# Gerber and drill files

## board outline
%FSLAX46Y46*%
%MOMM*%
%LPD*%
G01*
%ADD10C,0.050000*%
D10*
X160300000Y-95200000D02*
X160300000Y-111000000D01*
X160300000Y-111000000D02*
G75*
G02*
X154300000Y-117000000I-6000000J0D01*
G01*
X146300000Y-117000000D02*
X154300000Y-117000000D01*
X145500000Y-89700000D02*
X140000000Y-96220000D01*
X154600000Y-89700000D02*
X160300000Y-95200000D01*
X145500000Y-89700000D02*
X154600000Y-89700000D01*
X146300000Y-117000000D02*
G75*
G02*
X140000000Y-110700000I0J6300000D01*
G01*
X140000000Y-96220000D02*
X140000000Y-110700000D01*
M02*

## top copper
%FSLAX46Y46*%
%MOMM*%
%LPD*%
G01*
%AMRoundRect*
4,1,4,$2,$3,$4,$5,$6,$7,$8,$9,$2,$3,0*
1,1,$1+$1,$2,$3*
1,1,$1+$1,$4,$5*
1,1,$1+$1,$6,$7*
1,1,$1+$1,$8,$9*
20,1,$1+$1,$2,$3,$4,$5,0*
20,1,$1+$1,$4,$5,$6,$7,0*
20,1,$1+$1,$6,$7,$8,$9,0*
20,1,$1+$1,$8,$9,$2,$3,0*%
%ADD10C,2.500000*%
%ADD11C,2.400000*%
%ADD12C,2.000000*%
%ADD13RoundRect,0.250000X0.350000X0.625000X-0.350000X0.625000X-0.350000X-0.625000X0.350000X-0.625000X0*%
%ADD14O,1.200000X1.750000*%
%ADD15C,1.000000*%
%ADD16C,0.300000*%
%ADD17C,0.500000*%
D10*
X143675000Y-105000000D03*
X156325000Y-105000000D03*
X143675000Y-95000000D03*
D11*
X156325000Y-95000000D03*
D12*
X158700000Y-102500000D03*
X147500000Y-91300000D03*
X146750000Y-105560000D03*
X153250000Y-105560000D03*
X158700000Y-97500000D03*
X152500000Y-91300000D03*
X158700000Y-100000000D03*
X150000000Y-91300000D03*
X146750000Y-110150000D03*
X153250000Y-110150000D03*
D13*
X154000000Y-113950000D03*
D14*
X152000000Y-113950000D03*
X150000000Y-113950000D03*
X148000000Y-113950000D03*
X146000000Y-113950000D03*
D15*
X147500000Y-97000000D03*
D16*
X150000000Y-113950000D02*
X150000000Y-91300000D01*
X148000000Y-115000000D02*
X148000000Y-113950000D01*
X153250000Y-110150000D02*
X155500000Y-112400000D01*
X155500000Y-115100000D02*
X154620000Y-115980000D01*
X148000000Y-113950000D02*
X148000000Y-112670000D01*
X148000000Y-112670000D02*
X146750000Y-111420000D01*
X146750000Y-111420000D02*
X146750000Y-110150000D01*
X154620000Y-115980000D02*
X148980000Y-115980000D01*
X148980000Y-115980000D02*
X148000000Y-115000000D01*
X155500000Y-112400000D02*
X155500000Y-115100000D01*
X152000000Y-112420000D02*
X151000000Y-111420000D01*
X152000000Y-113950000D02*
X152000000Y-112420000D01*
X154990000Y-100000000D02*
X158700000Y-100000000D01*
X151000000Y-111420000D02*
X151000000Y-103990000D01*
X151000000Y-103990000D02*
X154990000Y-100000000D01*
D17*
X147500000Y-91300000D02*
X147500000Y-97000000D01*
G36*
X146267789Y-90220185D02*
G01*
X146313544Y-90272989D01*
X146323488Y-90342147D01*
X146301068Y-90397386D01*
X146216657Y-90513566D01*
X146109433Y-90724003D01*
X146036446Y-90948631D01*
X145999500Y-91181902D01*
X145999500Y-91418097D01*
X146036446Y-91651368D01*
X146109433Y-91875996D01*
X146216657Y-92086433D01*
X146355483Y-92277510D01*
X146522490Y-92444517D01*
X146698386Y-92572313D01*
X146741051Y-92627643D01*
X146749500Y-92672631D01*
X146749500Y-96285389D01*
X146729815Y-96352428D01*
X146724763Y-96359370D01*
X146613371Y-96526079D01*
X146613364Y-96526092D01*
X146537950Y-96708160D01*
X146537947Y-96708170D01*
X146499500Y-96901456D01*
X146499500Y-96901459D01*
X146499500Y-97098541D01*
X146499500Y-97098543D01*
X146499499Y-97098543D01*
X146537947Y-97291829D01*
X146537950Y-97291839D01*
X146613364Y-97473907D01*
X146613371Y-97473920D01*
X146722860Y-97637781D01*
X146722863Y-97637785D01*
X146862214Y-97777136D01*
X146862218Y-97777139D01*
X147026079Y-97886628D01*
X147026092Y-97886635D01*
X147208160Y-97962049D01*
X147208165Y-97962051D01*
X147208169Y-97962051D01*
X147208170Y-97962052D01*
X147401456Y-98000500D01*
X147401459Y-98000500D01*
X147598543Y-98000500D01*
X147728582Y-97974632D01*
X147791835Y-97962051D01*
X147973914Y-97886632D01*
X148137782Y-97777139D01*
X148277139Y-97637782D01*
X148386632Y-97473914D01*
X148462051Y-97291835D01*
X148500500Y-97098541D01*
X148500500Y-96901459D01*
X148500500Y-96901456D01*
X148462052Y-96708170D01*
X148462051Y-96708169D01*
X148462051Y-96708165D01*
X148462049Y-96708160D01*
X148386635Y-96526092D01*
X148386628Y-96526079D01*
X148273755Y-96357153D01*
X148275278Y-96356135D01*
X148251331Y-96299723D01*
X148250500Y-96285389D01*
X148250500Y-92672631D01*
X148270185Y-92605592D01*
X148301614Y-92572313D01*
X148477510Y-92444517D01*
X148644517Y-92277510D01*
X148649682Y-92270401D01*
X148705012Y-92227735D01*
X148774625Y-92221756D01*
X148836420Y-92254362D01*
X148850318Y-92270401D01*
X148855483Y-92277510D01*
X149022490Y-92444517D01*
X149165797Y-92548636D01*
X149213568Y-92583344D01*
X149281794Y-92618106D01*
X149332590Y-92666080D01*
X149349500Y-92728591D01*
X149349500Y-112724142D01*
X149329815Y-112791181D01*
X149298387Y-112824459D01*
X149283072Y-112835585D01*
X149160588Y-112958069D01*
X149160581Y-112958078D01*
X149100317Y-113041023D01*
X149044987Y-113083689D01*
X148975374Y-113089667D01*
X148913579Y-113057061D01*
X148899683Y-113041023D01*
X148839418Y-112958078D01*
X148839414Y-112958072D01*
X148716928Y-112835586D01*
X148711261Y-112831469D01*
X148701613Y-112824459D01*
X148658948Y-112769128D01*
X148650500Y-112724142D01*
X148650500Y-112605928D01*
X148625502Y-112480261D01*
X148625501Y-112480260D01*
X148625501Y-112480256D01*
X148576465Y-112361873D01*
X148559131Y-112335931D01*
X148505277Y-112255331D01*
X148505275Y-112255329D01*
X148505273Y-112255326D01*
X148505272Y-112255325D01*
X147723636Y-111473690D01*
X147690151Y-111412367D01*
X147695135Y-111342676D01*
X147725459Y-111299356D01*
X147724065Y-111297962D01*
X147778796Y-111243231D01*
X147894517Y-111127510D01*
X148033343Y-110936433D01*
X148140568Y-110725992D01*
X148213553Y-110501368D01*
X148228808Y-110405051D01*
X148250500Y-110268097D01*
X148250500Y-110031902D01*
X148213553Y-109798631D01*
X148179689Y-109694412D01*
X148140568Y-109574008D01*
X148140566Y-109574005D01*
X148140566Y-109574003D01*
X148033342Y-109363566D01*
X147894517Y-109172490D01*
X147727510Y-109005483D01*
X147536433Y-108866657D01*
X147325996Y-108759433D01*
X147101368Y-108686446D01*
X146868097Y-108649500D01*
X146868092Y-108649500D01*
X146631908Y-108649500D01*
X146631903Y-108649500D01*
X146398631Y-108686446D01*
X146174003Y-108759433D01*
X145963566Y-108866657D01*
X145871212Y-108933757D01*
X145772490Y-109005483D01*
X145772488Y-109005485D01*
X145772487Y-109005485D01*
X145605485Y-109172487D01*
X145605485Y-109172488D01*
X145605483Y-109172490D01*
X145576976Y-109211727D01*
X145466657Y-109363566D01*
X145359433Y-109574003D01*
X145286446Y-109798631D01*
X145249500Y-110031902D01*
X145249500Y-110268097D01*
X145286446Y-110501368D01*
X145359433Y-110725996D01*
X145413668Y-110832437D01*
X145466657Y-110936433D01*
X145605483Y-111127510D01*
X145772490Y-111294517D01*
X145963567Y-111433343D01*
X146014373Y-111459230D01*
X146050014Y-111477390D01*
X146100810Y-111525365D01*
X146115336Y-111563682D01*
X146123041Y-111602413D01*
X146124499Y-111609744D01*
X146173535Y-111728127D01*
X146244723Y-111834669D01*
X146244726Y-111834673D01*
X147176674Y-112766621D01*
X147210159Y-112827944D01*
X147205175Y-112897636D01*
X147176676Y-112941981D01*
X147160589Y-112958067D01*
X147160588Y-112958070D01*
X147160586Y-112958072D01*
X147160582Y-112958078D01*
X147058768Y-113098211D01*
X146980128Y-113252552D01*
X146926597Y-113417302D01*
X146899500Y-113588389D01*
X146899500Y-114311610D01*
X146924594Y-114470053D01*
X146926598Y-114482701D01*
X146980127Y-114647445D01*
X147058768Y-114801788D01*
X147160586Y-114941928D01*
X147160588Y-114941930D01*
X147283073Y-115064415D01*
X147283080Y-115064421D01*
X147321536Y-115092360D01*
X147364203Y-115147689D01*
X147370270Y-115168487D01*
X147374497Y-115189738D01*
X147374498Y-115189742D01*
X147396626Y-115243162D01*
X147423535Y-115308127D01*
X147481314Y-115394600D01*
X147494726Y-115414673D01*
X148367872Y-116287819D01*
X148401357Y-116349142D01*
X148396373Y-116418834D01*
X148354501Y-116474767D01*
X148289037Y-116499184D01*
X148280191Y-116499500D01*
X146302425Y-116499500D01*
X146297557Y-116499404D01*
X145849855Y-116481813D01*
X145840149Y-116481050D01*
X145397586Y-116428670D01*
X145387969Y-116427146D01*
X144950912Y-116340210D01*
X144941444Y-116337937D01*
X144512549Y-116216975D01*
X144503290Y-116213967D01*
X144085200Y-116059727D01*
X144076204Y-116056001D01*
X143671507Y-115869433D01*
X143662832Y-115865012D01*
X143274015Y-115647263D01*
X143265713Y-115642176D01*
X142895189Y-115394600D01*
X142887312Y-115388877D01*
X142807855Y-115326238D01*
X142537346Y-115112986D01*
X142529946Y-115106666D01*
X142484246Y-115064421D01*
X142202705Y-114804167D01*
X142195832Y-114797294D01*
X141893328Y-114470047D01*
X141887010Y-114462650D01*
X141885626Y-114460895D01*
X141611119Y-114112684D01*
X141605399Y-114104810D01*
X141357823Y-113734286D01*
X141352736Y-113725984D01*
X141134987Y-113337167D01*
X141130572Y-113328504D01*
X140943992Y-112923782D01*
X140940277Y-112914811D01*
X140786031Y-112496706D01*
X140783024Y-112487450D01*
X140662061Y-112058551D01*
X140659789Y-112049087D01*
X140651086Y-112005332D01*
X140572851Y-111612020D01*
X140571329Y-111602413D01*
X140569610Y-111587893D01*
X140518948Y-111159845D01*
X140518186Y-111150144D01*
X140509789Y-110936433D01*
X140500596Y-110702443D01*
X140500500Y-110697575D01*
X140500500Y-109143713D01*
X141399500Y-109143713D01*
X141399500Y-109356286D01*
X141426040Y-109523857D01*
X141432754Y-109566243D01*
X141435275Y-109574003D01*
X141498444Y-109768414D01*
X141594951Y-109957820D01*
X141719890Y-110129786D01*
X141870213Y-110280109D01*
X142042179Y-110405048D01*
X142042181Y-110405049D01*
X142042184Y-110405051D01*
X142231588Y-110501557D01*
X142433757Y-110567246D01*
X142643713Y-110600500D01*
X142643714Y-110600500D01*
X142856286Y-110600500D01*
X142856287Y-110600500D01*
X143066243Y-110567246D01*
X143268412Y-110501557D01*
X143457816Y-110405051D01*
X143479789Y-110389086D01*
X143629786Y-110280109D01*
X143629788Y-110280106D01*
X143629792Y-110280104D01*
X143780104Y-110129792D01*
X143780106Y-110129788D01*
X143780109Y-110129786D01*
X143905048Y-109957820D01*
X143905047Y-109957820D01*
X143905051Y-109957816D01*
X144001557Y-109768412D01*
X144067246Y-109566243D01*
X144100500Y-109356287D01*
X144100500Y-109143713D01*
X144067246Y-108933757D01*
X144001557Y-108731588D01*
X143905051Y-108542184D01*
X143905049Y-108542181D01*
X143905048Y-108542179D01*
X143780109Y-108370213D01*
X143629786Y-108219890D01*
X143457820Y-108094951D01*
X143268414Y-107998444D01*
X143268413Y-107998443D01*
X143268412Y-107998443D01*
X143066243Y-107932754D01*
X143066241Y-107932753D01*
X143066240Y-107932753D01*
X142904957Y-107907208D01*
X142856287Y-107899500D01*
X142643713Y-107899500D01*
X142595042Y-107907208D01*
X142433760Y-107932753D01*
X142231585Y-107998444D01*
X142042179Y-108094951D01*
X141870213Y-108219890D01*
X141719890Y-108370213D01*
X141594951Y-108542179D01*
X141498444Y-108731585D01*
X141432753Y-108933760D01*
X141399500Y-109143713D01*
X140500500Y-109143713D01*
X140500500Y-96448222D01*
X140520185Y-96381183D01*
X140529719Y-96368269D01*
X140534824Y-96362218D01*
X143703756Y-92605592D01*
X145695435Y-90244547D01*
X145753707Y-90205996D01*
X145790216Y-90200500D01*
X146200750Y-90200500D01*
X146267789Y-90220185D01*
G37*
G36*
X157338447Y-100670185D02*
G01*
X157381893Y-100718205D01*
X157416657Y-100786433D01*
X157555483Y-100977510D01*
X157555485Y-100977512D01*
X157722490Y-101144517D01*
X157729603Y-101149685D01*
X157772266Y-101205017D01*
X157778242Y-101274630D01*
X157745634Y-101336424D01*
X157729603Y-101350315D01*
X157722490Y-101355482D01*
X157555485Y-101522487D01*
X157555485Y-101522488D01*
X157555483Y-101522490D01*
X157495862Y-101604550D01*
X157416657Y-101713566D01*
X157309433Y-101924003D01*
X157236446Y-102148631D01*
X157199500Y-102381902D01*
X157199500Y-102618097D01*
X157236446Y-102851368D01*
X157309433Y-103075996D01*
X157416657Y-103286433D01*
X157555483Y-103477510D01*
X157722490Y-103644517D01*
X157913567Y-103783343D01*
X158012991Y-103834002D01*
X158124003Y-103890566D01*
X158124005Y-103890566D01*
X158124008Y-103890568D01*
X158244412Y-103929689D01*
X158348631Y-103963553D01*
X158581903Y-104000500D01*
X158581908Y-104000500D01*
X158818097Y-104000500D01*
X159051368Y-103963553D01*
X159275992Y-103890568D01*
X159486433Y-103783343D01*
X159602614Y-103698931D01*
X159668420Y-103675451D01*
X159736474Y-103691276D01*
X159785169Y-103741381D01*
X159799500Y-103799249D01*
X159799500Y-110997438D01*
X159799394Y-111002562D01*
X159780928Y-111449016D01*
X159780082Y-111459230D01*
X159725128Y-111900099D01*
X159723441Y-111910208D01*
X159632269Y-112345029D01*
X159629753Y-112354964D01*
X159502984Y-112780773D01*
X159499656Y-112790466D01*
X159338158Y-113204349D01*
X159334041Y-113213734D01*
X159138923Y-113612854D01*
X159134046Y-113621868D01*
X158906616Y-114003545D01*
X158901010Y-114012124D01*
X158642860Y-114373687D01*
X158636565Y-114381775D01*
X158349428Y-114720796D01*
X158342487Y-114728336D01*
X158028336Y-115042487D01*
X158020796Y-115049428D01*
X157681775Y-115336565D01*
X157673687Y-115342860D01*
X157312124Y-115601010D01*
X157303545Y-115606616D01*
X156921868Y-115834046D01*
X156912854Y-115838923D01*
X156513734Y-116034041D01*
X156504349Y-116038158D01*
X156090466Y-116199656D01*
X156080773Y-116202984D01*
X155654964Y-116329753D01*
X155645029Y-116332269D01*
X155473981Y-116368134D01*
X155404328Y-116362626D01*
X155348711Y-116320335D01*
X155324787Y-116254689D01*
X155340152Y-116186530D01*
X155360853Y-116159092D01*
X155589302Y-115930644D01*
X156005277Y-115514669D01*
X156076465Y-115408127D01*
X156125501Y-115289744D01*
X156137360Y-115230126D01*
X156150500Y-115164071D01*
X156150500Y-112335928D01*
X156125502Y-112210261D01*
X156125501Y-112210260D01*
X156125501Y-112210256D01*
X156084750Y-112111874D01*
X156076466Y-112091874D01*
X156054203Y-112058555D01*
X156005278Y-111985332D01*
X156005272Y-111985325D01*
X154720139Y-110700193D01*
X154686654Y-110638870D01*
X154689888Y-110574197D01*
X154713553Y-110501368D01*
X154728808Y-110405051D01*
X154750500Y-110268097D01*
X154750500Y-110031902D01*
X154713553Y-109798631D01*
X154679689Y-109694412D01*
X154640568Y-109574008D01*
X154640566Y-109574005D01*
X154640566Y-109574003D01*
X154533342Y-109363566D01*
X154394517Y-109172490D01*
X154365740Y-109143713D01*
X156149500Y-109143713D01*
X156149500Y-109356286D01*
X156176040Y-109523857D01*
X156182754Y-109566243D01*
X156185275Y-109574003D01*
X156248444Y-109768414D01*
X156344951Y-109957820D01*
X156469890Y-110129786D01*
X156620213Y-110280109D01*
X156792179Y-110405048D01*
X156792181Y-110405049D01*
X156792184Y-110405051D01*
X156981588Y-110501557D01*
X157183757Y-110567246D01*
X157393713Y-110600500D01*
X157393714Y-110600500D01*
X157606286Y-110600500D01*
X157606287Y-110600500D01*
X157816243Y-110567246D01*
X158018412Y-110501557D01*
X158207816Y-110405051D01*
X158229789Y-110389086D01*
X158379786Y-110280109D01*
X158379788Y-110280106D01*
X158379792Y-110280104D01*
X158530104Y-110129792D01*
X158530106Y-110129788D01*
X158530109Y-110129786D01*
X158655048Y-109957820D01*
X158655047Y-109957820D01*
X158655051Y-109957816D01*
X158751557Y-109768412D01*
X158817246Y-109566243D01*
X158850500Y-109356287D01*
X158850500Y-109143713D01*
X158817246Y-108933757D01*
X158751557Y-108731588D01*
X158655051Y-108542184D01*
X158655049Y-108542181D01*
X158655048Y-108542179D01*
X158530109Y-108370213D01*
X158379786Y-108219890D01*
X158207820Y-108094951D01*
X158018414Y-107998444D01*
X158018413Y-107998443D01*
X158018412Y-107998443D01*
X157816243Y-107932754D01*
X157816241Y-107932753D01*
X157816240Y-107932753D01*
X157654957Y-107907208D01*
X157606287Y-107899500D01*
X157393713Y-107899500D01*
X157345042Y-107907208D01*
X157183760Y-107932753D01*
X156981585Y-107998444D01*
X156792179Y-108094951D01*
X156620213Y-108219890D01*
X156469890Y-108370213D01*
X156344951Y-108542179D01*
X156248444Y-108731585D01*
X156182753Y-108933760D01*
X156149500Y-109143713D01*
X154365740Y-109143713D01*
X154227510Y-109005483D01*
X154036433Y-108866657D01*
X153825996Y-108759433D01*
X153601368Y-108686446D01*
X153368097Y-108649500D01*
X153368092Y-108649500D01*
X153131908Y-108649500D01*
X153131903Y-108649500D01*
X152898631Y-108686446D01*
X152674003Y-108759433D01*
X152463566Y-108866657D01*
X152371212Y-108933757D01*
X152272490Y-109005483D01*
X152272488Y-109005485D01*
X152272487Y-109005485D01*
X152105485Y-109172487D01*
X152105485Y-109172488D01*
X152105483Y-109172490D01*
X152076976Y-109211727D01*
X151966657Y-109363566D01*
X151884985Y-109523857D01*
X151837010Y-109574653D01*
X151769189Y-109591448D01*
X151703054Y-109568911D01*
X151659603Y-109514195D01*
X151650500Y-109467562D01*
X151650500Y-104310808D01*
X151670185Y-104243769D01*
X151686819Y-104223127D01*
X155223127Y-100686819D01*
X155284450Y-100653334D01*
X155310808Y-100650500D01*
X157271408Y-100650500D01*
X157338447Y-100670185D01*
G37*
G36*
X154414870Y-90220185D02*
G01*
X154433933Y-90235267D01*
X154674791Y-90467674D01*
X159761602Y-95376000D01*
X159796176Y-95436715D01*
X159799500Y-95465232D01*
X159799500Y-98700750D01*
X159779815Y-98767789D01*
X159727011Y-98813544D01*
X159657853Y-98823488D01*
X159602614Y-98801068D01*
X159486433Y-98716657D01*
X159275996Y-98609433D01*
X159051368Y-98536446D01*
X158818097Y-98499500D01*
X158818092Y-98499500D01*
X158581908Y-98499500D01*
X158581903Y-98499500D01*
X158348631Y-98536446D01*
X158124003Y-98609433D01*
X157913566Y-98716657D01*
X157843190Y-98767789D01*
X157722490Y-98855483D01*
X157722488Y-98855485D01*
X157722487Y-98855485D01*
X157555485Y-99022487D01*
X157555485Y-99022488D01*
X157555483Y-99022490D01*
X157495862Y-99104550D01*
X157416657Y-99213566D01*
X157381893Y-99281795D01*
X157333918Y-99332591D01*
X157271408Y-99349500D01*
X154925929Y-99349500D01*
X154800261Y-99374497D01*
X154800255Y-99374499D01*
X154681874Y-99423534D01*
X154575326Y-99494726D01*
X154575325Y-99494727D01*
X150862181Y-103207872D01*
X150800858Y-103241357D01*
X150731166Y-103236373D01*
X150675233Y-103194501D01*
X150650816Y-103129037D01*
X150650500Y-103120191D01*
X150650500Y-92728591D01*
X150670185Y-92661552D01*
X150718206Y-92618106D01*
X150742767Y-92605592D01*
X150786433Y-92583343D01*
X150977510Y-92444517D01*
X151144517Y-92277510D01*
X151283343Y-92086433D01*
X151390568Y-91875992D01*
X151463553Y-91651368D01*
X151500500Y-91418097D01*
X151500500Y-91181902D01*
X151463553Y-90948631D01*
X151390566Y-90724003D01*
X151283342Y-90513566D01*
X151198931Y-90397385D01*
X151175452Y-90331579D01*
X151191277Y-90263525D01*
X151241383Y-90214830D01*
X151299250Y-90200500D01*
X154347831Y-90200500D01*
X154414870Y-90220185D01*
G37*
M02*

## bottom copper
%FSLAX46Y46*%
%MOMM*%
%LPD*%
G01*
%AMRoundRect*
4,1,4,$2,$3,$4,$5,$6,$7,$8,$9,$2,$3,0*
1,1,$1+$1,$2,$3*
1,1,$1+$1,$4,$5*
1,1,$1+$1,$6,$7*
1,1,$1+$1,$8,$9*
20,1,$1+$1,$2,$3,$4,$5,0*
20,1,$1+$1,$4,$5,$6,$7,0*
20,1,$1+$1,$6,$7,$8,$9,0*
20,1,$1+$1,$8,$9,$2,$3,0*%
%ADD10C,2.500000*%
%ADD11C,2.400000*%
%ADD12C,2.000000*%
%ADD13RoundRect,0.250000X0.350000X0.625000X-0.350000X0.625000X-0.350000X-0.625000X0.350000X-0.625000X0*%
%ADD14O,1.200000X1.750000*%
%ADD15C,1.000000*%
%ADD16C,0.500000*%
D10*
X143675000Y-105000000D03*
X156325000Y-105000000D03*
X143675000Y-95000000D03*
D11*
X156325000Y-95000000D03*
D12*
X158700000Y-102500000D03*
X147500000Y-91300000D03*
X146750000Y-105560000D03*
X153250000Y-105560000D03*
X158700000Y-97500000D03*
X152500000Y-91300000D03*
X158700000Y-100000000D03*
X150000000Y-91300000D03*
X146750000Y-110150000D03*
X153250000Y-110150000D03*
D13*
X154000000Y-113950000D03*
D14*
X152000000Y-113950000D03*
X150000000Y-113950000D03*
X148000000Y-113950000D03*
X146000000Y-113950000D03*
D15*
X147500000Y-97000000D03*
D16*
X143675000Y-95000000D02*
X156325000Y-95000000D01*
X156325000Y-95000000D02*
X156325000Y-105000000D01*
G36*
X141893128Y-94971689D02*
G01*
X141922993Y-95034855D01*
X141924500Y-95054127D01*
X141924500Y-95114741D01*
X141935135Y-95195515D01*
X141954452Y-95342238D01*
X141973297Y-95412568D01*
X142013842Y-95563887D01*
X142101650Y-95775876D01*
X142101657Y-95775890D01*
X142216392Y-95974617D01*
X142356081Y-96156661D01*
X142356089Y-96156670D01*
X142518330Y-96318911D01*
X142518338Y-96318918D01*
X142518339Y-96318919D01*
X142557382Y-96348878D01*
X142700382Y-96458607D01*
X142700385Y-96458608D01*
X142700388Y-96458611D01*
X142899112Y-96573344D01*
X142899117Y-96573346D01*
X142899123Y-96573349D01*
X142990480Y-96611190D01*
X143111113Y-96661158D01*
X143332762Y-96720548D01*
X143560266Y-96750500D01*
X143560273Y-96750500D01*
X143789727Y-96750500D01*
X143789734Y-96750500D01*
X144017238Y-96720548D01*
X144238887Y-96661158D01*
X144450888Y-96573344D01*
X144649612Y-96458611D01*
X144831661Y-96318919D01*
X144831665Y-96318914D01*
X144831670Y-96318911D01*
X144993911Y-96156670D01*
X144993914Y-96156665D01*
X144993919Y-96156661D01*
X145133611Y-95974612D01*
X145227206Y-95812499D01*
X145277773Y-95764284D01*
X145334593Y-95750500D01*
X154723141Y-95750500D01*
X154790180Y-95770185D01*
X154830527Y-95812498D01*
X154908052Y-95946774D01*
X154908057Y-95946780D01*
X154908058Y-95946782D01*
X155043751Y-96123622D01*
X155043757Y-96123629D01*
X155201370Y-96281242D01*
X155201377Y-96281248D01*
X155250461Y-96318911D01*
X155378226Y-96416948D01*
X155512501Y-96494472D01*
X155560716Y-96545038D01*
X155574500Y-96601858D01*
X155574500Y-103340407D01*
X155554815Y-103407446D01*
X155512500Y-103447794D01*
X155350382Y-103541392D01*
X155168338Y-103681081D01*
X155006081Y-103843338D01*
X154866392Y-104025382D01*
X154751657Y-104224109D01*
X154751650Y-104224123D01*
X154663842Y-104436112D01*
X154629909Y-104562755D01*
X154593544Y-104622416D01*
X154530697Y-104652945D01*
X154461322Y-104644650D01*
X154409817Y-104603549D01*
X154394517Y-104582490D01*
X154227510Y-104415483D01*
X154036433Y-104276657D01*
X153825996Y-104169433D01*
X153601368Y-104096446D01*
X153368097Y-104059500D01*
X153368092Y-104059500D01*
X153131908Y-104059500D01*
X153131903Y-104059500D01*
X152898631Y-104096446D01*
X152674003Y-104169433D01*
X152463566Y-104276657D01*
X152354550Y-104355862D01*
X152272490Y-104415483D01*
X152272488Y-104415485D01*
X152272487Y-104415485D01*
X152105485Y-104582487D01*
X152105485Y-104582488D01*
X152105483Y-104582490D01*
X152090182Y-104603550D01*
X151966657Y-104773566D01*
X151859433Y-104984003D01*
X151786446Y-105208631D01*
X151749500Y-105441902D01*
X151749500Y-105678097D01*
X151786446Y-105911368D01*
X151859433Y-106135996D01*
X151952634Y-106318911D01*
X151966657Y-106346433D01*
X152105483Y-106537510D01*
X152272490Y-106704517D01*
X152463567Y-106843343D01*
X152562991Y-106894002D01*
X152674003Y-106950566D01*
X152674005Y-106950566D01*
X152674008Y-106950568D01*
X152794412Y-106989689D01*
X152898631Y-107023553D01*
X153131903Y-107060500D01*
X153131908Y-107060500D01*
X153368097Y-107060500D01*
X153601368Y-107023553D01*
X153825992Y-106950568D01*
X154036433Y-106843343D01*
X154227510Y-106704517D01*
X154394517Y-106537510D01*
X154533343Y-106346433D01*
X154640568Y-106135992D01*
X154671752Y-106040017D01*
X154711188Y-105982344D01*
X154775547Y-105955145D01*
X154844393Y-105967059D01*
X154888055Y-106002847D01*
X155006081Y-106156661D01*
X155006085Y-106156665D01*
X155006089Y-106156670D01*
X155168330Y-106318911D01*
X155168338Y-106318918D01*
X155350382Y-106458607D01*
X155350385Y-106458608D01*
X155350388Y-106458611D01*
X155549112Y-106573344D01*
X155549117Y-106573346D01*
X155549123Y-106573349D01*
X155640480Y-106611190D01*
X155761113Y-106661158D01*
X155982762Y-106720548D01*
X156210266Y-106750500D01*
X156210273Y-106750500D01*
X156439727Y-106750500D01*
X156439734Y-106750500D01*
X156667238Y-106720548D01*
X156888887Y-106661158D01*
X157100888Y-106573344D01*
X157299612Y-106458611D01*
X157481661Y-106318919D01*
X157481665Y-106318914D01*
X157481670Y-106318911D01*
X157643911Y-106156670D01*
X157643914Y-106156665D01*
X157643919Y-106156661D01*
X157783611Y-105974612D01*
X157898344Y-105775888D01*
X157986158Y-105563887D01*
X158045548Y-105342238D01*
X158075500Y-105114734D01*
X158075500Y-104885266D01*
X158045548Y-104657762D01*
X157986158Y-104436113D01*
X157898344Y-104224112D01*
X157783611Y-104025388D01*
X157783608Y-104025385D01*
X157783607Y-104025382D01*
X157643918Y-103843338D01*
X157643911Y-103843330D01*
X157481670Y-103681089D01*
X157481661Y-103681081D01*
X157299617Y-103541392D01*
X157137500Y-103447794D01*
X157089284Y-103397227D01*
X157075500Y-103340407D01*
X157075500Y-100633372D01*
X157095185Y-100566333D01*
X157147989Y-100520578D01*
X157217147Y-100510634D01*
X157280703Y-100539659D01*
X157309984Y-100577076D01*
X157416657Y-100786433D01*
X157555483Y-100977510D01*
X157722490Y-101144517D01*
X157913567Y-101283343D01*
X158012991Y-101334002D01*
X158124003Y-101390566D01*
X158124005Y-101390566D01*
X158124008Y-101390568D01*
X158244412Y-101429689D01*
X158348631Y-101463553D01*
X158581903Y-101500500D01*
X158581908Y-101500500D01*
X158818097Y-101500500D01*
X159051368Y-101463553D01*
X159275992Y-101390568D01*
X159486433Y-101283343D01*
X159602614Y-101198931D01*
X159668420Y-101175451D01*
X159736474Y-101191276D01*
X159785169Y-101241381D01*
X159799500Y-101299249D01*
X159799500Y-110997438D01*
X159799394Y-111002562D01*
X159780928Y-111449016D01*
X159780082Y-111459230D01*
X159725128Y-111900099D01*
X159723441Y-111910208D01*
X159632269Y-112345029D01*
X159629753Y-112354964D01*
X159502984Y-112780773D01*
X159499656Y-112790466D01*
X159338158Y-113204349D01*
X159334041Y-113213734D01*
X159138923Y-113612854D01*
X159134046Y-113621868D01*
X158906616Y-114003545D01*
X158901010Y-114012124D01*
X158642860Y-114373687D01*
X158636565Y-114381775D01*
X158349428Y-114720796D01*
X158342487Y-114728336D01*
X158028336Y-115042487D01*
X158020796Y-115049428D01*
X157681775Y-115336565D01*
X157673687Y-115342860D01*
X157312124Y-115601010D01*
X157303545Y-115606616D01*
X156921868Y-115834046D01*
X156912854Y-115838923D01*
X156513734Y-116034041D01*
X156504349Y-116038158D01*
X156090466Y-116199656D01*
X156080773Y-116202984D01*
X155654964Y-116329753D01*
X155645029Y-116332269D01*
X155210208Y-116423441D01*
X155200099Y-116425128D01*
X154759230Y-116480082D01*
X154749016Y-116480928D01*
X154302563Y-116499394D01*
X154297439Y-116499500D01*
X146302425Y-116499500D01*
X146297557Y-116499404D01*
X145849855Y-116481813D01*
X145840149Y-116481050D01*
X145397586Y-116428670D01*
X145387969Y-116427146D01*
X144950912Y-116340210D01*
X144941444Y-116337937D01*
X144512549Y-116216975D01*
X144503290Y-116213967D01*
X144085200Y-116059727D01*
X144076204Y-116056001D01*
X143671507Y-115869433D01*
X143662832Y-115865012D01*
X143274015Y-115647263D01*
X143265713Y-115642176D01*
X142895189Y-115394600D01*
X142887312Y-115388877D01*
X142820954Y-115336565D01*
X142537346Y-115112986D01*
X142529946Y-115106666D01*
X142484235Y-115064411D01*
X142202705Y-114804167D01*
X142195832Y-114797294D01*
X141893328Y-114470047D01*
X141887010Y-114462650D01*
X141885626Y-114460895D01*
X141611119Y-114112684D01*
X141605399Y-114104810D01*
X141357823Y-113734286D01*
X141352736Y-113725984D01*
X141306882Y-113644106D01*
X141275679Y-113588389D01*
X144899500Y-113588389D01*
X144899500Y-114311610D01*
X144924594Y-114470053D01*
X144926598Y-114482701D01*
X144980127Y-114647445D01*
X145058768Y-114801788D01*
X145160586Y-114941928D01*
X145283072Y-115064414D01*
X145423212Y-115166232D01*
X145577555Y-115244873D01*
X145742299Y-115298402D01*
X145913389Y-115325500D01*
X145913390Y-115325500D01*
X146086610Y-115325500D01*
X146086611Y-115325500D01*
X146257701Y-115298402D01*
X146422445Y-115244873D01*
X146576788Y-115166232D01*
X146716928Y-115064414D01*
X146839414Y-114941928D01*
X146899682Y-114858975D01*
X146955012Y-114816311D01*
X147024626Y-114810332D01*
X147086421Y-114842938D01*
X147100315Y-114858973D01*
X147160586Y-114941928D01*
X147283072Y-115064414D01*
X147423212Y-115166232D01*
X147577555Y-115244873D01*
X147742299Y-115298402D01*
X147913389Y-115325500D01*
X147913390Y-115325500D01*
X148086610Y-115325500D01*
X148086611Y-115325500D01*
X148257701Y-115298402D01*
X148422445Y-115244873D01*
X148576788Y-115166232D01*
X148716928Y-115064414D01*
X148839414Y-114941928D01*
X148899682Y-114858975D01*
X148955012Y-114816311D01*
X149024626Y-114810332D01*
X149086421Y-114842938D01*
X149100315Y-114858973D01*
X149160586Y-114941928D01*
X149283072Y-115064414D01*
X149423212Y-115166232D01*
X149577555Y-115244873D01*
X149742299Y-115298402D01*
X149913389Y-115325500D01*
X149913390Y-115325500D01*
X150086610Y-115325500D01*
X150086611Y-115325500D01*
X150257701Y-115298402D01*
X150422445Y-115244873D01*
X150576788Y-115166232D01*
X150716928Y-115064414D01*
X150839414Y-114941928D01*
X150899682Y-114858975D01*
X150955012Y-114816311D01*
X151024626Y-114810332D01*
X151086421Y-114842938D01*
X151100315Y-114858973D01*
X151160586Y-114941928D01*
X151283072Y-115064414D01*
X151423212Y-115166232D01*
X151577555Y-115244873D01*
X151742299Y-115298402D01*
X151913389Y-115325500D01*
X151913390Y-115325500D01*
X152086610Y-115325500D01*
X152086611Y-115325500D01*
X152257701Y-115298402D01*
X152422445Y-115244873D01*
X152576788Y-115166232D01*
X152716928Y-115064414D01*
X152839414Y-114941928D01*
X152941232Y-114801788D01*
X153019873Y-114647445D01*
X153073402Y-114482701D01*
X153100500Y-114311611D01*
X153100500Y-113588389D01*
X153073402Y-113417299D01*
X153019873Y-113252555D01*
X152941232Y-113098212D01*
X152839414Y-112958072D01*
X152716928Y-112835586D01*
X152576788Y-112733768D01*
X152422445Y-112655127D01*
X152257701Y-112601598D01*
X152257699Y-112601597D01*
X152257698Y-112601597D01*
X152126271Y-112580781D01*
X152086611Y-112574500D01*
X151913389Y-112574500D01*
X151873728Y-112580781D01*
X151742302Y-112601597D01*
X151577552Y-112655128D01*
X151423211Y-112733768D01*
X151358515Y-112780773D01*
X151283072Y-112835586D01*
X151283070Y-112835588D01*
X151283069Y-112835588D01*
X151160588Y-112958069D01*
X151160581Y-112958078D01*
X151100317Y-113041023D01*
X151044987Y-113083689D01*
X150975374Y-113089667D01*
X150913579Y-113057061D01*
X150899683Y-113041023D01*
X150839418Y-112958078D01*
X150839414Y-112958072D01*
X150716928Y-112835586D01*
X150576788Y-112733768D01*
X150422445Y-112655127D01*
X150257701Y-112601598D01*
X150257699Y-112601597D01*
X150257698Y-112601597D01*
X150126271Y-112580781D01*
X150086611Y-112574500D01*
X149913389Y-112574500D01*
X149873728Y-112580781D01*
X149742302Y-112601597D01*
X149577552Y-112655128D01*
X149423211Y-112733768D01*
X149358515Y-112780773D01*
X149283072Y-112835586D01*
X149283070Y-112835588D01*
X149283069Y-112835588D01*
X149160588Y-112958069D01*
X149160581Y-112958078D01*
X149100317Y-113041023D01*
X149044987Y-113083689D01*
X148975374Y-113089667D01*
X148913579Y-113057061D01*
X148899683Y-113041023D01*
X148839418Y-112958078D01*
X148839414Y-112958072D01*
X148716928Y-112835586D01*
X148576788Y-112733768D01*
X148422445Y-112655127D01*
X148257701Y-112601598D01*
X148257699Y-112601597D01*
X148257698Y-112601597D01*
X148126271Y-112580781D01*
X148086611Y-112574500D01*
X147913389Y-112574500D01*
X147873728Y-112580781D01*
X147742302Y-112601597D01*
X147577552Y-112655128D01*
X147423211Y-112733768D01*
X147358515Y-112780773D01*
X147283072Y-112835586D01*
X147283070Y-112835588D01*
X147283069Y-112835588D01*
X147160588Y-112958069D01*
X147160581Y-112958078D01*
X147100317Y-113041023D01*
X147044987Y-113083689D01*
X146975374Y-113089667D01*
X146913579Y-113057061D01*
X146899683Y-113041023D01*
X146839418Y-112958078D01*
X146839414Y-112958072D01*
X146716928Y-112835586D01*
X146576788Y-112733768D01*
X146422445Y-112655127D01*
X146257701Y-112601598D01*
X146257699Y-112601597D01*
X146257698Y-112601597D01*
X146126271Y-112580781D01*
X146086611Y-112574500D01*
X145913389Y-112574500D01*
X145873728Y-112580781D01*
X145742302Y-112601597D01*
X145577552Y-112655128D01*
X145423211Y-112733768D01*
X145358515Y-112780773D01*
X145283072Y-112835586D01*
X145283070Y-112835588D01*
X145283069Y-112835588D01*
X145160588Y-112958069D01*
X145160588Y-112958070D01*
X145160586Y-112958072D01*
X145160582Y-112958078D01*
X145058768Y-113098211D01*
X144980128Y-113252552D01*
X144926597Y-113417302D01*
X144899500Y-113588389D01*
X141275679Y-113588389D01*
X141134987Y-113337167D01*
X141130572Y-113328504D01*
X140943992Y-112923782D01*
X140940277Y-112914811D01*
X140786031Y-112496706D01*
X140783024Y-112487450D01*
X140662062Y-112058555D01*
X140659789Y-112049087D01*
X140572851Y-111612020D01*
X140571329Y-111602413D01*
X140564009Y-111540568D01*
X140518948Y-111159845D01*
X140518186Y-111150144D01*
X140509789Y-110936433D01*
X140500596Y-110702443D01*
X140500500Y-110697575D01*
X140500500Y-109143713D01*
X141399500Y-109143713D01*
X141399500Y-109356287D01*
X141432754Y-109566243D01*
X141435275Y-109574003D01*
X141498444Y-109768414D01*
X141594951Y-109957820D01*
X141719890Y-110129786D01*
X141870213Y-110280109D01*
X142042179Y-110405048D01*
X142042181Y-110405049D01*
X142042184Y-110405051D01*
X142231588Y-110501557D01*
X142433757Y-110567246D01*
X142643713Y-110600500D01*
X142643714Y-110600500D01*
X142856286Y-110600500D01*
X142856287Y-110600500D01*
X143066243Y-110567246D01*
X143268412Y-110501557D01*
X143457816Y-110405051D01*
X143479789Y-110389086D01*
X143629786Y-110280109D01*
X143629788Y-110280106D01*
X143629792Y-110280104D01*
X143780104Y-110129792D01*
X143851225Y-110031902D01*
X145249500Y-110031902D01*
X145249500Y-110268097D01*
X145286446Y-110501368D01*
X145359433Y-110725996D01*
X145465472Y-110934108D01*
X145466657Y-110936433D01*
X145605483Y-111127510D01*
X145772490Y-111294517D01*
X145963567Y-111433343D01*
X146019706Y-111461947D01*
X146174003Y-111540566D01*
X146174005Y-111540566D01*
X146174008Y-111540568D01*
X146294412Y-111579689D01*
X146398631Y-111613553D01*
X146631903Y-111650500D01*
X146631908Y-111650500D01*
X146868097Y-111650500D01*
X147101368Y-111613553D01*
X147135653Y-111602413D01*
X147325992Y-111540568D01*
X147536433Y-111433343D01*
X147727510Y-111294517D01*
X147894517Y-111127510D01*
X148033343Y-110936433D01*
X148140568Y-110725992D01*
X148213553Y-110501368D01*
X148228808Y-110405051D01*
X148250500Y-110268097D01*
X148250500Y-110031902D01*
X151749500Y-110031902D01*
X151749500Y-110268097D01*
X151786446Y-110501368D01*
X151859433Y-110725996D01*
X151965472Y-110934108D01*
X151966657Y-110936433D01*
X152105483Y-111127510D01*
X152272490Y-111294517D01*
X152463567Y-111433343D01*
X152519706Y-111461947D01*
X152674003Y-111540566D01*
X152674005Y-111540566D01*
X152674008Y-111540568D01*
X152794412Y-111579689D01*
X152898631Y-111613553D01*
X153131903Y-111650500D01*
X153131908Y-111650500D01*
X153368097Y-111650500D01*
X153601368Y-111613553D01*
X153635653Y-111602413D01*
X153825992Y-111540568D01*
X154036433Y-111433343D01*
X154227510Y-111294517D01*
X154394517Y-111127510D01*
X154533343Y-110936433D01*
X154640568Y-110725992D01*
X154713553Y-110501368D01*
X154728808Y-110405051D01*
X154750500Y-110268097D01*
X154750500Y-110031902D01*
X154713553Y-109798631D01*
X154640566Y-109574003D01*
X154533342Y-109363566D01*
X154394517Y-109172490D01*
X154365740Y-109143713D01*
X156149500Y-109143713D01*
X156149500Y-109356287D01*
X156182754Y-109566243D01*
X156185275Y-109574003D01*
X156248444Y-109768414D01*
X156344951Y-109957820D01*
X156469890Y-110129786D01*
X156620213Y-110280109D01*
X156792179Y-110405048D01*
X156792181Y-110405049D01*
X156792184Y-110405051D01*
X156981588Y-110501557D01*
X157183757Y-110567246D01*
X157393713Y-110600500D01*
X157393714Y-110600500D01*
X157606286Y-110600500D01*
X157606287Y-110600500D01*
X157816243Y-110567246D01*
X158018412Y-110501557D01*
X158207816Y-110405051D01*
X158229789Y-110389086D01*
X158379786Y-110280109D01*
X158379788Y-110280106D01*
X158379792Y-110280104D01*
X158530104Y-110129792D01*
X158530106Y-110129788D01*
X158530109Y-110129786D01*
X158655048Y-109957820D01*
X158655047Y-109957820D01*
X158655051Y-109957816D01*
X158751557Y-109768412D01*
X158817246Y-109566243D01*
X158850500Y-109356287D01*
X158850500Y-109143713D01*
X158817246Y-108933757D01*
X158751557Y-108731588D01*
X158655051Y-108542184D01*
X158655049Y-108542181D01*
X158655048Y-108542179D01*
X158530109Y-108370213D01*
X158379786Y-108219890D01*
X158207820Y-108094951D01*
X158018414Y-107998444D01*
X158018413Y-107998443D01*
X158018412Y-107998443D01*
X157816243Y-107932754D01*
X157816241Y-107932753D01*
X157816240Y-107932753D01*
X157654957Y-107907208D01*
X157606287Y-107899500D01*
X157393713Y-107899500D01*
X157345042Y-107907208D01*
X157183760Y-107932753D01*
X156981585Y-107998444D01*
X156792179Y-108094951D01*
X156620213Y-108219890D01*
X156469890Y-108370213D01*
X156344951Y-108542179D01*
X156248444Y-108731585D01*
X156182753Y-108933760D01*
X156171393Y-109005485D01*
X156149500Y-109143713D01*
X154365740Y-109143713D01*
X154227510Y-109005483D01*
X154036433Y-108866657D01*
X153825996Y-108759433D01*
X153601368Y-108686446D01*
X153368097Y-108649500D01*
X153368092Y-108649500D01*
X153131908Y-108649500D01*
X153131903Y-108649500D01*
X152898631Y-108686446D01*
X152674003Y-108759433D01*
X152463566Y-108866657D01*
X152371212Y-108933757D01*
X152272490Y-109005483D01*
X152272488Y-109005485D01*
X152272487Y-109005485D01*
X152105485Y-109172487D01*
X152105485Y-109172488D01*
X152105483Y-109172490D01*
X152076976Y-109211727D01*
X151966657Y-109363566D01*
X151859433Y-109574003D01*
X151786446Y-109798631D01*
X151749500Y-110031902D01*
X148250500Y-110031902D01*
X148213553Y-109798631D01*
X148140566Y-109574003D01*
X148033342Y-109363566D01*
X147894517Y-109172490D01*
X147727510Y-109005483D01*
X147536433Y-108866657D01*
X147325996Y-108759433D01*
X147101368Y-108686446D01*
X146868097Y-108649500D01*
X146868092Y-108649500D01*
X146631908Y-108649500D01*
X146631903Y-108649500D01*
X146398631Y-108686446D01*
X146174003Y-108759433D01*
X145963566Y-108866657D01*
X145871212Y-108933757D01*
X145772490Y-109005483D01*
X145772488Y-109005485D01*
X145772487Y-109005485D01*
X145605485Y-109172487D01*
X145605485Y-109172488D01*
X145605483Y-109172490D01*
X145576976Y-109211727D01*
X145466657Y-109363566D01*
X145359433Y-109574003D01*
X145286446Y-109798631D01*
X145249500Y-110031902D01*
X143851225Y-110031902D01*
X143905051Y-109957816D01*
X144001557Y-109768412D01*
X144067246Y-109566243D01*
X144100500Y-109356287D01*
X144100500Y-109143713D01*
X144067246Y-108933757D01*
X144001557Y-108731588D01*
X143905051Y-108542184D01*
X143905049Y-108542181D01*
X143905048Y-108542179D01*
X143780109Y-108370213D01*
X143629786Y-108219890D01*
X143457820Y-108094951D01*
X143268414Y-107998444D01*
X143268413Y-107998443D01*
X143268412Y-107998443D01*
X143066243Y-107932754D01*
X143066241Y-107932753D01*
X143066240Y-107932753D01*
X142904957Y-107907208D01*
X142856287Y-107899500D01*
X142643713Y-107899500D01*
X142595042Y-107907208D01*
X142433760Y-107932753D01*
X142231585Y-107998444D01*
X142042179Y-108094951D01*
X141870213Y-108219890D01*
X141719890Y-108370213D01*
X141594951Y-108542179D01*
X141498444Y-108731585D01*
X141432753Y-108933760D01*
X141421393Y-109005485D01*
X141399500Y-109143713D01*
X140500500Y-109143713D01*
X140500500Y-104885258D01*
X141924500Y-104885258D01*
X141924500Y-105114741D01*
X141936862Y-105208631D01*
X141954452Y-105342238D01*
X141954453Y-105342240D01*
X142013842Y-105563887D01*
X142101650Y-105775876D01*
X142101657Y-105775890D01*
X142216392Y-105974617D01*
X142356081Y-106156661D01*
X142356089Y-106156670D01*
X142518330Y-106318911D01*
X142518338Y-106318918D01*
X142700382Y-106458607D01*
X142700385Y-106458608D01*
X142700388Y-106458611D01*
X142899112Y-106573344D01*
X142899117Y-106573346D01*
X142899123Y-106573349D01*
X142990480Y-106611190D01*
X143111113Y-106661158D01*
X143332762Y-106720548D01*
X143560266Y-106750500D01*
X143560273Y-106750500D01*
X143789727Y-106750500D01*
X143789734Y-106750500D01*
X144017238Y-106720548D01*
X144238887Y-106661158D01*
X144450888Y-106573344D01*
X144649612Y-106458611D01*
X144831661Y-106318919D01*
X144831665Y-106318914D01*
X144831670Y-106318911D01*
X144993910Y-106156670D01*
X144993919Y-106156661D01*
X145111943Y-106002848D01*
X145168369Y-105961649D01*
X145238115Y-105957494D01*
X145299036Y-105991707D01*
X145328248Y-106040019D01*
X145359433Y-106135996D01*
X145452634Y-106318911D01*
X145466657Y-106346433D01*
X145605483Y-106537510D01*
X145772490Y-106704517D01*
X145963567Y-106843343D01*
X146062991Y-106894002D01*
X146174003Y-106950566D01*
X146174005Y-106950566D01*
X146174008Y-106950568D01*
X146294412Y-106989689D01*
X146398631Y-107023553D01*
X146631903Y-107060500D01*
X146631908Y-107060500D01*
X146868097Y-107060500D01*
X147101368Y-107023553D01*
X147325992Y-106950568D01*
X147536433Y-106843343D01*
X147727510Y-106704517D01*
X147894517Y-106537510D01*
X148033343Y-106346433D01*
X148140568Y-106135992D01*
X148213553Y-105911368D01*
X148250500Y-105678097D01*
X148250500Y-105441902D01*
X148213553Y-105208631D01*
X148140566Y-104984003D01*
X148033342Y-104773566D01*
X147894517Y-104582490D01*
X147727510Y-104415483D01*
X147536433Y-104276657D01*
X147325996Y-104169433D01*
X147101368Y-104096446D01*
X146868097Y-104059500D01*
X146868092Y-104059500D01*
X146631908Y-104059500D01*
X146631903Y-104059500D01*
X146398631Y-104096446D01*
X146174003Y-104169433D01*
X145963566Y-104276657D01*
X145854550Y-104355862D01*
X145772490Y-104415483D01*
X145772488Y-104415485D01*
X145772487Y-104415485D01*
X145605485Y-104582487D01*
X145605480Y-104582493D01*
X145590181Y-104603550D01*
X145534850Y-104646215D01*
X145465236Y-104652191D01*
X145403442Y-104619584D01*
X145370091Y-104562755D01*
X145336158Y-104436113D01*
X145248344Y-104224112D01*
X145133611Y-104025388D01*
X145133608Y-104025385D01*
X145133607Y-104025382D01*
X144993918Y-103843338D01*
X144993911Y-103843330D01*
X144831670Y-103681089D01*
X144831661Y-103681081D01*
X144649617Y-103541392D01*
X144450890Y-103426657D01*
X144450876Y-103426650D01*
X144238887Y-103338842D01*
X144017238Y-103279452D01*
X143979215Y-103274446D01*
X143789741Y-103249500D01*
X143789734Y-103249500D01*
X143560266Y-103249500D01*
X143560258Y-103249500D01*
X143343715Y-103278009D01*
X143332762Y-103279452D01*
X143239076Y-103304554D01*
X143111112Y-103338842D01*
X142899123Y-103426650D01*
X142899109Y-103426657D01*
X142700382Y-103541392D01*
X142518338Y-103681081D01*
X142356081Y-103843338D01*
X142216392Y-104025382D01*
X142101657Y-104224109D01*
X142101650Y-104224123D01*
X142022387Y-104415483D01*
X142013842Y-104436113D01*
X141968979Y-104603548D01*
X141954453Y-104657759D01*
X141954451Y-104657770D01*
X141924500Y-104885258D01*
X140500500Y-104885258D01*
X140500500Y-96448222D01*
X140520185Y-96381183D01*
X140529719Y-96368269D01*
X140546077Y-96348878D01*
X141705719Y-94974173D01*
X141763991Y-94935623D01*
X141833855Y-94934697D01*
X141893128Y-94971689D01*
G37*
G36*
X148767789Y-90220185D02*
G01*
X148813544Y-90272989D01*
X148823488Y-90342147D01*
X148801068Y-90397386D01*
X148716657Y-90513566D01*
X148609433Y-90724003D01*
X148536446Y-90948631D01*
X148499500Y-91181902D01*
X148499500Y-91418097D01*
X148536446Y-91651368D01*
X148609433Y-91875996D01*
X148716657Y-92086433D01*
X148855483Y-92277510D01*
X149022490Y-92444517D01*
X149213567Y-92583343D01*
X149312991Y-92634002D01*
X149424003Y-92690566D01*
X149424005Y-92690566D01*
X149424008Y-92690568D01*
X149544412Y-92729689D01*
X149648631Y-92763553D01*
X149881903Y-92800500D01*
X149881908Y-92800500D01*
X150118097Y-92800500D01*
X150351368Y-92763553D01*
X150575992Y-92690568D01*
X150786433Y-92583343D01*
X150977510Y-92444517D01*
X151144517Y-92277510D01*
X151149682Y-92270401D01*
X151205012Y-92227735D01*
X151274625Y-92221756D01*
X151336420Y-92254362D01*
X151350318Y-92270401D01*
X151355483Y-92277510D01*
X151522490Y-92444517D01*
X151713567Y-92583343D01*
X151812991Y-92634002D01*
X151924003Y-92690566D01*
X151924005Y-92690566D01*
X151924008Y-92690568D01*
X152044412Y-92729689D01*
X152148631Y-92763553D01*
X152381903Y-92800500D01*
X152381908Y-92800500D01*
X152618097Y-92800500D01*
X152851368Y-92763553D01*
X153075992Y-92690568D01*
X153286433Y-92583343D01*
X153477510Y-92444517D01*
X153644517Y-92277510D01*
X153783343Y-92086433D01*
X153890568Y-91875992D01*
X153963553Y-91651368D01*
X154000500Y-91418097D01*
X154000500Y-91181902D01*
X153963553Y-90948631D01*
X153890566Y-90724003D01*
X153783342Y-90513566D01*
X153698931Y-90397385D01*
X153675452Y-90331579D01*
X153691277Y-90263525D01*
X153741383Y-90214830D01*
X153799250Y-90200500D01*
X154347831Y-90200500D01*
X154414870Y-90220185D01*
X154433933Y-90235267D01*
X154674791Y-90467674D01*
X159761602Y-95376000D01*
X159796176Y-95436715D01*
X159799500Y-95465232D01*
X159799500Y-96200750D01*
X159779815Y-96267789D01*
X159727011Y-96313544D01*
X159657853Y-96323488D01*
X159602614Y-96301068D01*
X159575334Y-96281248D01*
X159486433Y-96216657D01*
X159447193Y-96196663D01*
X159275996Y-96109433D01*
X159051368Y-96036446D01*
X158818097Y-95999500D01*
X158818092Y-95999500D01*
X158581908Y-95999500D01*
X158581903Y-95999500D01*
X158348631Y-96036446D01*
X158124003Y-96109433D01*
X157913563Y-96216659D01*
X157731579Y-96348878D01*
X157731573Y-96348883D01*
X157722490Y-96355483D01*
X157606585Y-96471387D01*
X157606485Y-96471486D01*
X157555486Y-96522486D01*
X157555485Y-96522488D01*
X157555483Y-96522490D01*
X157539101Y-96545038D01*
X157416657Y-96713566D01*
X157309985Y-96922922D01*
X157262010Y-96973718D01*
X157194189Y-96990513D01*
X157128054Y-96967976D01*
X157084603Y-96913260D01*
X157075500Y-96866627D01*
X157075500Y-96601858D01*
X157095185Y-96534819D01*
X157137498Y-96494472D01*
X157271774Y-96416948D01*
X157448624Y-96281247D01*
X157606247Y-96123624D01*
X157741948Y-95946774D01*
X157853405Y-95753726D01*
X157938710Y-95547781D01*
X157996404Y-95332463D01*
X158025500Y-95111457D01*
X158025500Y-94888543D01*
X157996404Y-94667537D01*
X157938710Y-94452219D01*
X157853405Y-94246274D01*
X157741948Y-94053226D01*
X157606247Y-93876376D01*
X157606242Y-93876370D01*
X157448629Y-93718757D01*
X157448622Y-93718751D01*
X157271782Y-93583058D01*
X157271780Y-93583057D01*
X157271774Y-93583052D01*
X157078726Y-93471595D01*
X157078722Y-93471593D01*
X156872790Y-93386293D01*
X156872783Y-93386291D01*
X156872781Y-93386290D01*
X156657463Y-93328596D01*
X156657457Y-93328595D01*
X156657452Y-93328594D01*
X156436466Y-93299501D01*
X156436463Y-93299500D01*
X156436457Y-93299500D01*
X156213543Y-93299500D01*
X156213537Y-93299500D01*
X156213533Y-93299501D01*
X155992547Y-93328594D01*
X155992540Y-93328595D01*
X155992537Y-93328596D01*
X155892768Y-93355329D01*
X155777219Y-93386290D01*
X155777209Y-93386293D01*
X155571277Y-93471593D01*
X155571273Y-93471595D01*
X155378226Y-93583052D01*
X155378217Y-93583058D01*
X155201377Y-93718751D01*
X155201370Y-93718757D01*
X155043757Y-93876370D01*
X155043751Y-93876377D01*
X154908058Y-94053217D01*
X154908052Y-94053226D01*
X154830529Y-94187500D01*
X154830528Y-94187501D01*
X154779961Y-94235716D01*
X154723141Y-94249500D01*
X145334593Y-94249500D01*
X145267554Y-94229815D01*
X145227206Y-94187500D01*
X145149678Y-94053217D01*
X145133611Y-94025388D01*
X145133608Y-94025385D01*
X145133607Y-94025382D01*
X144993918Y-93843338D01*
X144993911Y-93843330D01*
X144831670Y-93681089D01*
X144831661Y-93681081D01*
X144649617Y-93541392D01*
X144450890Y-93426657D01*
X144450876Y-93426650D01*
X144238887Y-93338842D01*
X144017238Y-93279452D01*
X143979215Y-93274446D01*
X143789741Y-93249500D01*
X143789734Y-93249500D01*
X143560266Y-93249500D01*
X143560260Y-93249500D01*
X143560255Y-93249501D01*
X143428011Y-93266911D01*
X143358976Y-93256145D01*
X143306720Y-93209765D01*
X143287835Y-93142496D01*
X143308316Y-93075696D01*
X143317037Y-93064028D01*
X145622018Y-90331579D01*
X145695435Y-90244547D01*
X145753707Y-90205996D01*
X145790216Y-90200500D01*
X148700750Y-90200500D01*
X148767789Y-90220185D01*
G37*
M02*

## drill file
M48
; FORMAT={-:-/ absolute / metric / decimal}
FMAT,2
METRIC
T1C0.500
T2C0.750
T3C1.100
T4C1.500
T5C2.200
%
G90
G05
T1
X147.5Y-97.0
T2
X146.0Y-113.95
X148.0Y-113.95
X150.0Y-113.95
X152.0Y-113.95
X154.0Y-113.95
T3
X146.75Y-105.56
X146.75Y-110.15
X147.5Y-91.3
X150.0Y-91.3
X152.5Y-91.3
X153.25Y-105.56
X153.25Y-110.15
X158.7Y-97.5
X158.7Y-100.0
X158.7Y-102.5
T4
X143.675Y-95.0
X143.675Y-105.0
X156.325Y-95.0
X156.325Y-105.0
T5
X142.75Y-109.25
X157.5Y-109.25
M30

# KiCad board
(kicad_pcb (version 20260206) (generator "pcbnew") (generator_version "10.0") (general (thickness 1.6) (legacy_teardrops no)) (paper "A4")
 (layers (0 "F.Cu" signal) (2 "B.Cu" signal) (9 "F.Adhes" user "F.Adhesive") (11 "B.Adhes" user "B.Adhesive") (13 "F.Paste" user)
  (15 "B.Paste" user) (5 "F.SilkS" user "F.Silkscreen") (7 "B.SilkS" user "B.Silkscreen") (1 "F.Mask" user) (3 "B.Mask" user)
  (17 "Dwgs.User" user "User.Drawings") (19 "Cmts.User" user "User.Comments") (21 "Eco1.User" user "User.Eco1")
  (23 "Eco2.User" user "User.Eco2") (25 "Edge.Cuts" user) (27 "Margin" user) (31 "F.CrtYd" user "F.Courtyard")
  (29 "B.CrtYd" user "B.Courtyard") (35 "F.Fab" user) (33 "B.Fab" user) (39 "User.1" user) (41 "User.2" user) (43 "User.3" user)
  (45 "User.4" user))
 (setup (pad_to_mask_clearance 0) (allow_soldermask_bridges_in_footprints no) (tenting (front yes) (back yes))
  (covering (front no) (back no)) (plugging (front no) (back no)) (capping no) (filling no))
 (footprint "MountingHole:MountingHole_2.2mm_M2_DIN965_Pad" (layer "F.Cu") (at 157.5 109.25)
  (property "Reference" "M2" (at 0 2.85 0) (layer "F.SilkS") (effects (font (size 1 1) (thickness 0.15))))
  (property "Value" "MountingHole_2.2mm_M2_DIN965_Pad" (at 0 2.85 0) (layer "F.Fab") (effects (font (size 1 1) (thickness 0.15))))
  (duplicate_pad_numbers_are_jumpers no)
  (pad "" np_thru_hole circle (at 0 0) (size 2.2 3.8) (drill 2.2) (layers "*.Cu" "*.Mask") (zone_connect 2)))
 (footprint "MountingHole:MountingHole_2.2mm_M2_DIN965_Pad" (layer "F.Cu") (at 142.75 109.25)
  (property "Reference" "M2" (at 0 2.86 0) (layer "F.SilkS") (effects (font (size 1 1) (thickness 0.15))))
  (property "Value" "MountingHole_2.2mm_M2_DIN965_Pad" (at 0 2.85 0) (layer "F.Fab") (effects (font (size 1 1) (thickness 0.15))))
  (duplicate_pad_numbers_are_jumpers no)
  (pad "" np_thru_hole circle (at 0 0) (size 2.2 3.8) (drill 2.2) (layers "*.Cu" "*.Mask") (zone_connect 2)))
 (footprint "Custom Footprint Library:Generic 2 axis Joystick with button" (layer "F.Cu") (at 150 100 90)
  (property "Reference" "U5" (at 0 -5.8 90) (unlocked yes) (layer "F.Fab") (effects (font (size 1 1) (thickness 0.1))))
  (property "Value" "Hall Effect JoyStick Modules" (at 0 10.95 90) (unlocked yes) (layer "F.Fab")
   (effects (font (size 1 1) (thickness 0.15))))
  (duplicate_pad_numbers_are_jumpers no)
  (pad "" thru_hole circle (at -5 -6.325 90) (size 2.5 2.5) (drill 1.5) (layers "*.Cu" "*.Mask") (remove_unused_layers no) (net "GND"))
  (pad "" thru_hole circle (at -5 6.325 90) (size 2.5 2.5) (drill 1.5) (layers "*.Cu" "*.Mask") (remove_unused_layers no) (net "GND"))
  (pad "" thru_hole circle (at 5 -6.325 90) (size 2.5 2.5) (drill 1.5) (layers "*.Cu" "*.Mask") (remove_unused_layers no) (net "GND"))
  (pad "" thru_hole circle (at 5 6.325 90) (size 2.4 2.4) (drill 1.5) (layers "*.Cu" "*.Mask") (remove_unused_layers no) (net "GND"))
  (pad "1" thru_hole circle (at -2.5 8.7 90) (size 2 2) (drill 1.1) (layers "*.Cu" "*.Mask") (remove_unused_layers no) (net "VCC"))
  (pad "1" thru_hole circle (at 8.7 -2.5 90) (size 2 2) (drill 1.1) (layers "*.Cu" "*.Mask") (remove_unused_layers no) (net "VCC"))
  (pad "2" thru_hole circle (at -5.56 -3.25 90) (size 2 2) (drill 1.1) (layers "*.Cu" "*.Mask") (remove_unused_layers no) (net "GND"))
  (pad "2" thru_hole circle (at -5.56 3.25 90) (size 2 2) (drill 1.1) (layers "*.Cu" "*.Mask") (remove_unused_layers no) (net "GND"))
  (pad "2" thru_hole circle (at 2.5 8.7 90) (size 2 2) (drill 1.1) (layers "*.Cu" "*.Mask") (remove_unused_layers no) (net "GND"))
  (pad "2" thru_hole circle (at 8.7 2.5 90) (size 2 2) (drill 1.1) (layers "*.Cu" "*.Mask") (remove_unused_layers no) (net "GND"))
  (pad "3" thru_hole circle (at 0 8.7 90) (size 2 2) (drill 1.1) (layers "*.Cu" "*.Mask") (remove_unused_layers no) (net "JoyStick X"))
  (pad "4" thru_hole circle (at 8.7 0 90) (size 2 2) (drill 1.1) (layers "*.Cu" "*.Mask") (remove_unused_layers no) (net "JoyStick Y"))
  (pad "5" thru_hole circle (at -10.15 -3.25 90) (size 2 2) (drill 1.1) (layers "*.Cu" "*.Mask") (remove_unused_layers no)
   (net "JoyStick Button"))
  (pad "5" thru_hole circle (at -10.15 3.25 90) (size 2 2) (drill 1.1) (layers "*.Cu" "*.Mask") (remove_unused_layers no)
   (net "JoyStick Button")))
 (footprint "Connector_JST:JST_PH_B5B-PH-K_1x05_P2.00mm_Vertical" (layer "B.Cu") (at 154 113.95 180)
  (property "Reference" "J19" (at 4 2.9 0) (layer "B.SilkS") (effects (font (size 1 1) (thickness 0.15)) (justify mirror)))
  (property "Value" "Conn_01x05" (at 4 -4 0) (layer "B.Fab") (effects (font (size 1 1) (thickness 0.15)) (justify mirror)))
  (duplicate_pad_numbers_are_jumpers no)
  (pad "1" thru_hole roundrect (at 0 0 180) (size 1.2 1.75) (drill 0.75) (layers "*.Cu" "*.Mask") (remove_unused_layers no)
   (roundrect_rratio 0.208333) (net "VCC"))
  (pad "2" thru_hole oval (at 2 0 180) (size 1.2 1.75) (drill 0.75) (layers "*.Cu" "*.Mask") (remove_unused_layers no) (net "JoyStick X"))
  (pad "3" thru_hole oval (at 4 0 180) (size 1.2 1.75) (drill 0.75) (layers "*.Cu" "*.Mask") (remove_unused_layers no) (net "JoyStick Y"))
  (pad "4" thru_hole oval (at 6 0 180) (size 1.2 1.75) (drill 0.75) (layers "*.Cu" "*.Mask") (remove_unused_layers no)
   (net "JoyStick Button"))
  (pad "5" thru_hole oval (at 8 0 180) (size 1.2 1.75) (drill 0.75) (layers "*.Cu" "*.Mask") (remove_unused_layers no) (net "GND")))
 (gr_line (start 140 96.22) (end 140 110.7) (stroke (width 0.05) (type default)) (layer "Edge.Cuts"))
 (gr_line (start 145.5 89.7) (end 140 96.22) (stroke (width 0.05) (type default)) (layer "Edge.Cuts"))
 (gr_line (start 145.5 89.7) (end 154.6 89.7) (stroke (width 0.05) (type default)) (layer "Edge.Cuts"))
 (gr_arc (start 146.3 117) (mid 141.845227 115.154773) (end 140 110.7) (stroke (width 0.05) (type default)) (layer "Edge.Cuts"))
 (gr_line (start 146.3 117) (end 154.3 117) (stroke (width 0.05) (type default)) (layer "Edge.Cuts"))
 (gr_line (start 154.6 89.7) (end 160.3 95.2) (stroke (width 0.05) (type default)) (layer "Edge.Cuts"))
 (gr_line (start 160.3 95.2) (end 160.3 111) (stroke (width 0.05) (type default)) (layer "Edge.Cuts"))
 (gr_arc (start 160.3 111) (mid 158.542641 115.242641) (end 154.3 117) (stroke (width 0.05) (type default)) (layer "Edge.Cuts"))
 (segment (start 143.675 95) (end 156.325 95) (width 0.5) (layer "B.Cu") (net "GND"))
 (segment (start 156.325 95) (end 156.325 105) (width 0.5) (layer "B.Cu") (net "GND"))
 (segment (start 150 113.95) (end 150 91.3) (width 0.3) (layer "F.Cu") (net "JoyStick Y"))
 (segment (start 148 115) (end 148 113.95) (width 0.3) (layer "F.Cu") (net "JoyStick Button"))
 (segment (start 153.25 110.15) (end 155.5 112.4) (width 0.3) (layer "F.Cu") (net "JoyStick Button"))
 (segment (start 155.5 115.1) (end 154.62 115.98) (width 0.3) (layer "F.Cu") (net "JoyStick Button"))
 (segment (start 148 113.95) (end 148 112.67) (width 0.3) (layer "F.Cu") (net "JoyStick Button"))
 (segment (start 148 112.67) (end 146.75 111.42) (width 0.3) (layer "F.Cu") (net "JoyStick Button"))
 (segment (start 146.75 111.42) (end 146.75 110.15) (width 0.3) (layer "F.Cu") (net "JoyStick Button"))
 (segment (start 154.62 115.98) (end 148.98 115.98) (width 0.3) (layer "F.Cu") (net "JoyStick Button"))
 (segment (start 148.98 115.98) (end 148 115) (width 0.3) (layer "F.Cu") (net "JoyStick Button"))
 (segment (start 155.5 112.4) (end 155.5 115.1) (width 0.3) (layer "F.Cu") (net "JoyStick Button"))
 (segment (start 152 112.42) (end 151 111.42) (width 0.3) (layer "F.Cu") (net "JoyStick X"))
 (segment (start 152 113.95) (end 152 112.42) (width 0.3) (layer "F.Cu") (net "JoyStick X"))
 (segment (start 154.99 100) (end 158.7 100) (width 0.3) (layer "F.Cu") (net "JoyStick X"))
 (segment (start 151 111.42) (end 151 103.99) (width 0.3) (layer "F.Cu") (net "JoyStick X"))
 (segment (start 151 103.99) (end 154.99 100) (width 0.3) (layer "F.Cu") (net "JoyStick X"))
 (segment (start 147.5 91.3) (end 147.5 97) (width 0.5) (layer "F.Cu") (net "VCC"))
 (via (at 147.5 97) (size 1) (drill 0.5) (layers "F.Cu" "B.Cu") (capping no) (covering (front no) (back no)) (plugging (front no) (back no))
  (filling no) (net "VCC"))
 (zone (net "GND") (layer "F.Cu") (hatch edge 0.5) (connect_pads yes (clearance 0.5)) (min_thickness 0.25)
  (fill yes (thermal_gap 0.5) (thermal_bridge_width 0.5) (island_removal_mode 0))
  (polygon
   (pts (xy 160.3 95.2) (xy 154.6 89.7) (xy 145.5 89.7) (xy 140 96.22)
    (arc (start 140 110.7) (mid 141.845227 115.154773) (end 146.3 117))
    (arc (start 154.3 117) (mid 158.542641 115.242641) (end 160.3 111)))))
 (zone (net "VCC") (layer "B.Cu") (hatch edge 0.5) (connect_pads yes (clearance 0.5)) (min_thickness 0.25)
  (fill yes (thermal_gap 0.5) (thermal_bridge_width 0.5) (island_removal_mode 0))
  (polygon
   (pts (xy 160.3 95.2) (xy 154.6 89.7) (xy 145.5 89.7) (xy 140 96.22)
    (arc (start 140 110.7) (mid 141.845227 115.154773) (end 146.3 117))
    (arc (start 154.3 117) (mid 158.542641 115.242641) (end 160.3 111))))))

